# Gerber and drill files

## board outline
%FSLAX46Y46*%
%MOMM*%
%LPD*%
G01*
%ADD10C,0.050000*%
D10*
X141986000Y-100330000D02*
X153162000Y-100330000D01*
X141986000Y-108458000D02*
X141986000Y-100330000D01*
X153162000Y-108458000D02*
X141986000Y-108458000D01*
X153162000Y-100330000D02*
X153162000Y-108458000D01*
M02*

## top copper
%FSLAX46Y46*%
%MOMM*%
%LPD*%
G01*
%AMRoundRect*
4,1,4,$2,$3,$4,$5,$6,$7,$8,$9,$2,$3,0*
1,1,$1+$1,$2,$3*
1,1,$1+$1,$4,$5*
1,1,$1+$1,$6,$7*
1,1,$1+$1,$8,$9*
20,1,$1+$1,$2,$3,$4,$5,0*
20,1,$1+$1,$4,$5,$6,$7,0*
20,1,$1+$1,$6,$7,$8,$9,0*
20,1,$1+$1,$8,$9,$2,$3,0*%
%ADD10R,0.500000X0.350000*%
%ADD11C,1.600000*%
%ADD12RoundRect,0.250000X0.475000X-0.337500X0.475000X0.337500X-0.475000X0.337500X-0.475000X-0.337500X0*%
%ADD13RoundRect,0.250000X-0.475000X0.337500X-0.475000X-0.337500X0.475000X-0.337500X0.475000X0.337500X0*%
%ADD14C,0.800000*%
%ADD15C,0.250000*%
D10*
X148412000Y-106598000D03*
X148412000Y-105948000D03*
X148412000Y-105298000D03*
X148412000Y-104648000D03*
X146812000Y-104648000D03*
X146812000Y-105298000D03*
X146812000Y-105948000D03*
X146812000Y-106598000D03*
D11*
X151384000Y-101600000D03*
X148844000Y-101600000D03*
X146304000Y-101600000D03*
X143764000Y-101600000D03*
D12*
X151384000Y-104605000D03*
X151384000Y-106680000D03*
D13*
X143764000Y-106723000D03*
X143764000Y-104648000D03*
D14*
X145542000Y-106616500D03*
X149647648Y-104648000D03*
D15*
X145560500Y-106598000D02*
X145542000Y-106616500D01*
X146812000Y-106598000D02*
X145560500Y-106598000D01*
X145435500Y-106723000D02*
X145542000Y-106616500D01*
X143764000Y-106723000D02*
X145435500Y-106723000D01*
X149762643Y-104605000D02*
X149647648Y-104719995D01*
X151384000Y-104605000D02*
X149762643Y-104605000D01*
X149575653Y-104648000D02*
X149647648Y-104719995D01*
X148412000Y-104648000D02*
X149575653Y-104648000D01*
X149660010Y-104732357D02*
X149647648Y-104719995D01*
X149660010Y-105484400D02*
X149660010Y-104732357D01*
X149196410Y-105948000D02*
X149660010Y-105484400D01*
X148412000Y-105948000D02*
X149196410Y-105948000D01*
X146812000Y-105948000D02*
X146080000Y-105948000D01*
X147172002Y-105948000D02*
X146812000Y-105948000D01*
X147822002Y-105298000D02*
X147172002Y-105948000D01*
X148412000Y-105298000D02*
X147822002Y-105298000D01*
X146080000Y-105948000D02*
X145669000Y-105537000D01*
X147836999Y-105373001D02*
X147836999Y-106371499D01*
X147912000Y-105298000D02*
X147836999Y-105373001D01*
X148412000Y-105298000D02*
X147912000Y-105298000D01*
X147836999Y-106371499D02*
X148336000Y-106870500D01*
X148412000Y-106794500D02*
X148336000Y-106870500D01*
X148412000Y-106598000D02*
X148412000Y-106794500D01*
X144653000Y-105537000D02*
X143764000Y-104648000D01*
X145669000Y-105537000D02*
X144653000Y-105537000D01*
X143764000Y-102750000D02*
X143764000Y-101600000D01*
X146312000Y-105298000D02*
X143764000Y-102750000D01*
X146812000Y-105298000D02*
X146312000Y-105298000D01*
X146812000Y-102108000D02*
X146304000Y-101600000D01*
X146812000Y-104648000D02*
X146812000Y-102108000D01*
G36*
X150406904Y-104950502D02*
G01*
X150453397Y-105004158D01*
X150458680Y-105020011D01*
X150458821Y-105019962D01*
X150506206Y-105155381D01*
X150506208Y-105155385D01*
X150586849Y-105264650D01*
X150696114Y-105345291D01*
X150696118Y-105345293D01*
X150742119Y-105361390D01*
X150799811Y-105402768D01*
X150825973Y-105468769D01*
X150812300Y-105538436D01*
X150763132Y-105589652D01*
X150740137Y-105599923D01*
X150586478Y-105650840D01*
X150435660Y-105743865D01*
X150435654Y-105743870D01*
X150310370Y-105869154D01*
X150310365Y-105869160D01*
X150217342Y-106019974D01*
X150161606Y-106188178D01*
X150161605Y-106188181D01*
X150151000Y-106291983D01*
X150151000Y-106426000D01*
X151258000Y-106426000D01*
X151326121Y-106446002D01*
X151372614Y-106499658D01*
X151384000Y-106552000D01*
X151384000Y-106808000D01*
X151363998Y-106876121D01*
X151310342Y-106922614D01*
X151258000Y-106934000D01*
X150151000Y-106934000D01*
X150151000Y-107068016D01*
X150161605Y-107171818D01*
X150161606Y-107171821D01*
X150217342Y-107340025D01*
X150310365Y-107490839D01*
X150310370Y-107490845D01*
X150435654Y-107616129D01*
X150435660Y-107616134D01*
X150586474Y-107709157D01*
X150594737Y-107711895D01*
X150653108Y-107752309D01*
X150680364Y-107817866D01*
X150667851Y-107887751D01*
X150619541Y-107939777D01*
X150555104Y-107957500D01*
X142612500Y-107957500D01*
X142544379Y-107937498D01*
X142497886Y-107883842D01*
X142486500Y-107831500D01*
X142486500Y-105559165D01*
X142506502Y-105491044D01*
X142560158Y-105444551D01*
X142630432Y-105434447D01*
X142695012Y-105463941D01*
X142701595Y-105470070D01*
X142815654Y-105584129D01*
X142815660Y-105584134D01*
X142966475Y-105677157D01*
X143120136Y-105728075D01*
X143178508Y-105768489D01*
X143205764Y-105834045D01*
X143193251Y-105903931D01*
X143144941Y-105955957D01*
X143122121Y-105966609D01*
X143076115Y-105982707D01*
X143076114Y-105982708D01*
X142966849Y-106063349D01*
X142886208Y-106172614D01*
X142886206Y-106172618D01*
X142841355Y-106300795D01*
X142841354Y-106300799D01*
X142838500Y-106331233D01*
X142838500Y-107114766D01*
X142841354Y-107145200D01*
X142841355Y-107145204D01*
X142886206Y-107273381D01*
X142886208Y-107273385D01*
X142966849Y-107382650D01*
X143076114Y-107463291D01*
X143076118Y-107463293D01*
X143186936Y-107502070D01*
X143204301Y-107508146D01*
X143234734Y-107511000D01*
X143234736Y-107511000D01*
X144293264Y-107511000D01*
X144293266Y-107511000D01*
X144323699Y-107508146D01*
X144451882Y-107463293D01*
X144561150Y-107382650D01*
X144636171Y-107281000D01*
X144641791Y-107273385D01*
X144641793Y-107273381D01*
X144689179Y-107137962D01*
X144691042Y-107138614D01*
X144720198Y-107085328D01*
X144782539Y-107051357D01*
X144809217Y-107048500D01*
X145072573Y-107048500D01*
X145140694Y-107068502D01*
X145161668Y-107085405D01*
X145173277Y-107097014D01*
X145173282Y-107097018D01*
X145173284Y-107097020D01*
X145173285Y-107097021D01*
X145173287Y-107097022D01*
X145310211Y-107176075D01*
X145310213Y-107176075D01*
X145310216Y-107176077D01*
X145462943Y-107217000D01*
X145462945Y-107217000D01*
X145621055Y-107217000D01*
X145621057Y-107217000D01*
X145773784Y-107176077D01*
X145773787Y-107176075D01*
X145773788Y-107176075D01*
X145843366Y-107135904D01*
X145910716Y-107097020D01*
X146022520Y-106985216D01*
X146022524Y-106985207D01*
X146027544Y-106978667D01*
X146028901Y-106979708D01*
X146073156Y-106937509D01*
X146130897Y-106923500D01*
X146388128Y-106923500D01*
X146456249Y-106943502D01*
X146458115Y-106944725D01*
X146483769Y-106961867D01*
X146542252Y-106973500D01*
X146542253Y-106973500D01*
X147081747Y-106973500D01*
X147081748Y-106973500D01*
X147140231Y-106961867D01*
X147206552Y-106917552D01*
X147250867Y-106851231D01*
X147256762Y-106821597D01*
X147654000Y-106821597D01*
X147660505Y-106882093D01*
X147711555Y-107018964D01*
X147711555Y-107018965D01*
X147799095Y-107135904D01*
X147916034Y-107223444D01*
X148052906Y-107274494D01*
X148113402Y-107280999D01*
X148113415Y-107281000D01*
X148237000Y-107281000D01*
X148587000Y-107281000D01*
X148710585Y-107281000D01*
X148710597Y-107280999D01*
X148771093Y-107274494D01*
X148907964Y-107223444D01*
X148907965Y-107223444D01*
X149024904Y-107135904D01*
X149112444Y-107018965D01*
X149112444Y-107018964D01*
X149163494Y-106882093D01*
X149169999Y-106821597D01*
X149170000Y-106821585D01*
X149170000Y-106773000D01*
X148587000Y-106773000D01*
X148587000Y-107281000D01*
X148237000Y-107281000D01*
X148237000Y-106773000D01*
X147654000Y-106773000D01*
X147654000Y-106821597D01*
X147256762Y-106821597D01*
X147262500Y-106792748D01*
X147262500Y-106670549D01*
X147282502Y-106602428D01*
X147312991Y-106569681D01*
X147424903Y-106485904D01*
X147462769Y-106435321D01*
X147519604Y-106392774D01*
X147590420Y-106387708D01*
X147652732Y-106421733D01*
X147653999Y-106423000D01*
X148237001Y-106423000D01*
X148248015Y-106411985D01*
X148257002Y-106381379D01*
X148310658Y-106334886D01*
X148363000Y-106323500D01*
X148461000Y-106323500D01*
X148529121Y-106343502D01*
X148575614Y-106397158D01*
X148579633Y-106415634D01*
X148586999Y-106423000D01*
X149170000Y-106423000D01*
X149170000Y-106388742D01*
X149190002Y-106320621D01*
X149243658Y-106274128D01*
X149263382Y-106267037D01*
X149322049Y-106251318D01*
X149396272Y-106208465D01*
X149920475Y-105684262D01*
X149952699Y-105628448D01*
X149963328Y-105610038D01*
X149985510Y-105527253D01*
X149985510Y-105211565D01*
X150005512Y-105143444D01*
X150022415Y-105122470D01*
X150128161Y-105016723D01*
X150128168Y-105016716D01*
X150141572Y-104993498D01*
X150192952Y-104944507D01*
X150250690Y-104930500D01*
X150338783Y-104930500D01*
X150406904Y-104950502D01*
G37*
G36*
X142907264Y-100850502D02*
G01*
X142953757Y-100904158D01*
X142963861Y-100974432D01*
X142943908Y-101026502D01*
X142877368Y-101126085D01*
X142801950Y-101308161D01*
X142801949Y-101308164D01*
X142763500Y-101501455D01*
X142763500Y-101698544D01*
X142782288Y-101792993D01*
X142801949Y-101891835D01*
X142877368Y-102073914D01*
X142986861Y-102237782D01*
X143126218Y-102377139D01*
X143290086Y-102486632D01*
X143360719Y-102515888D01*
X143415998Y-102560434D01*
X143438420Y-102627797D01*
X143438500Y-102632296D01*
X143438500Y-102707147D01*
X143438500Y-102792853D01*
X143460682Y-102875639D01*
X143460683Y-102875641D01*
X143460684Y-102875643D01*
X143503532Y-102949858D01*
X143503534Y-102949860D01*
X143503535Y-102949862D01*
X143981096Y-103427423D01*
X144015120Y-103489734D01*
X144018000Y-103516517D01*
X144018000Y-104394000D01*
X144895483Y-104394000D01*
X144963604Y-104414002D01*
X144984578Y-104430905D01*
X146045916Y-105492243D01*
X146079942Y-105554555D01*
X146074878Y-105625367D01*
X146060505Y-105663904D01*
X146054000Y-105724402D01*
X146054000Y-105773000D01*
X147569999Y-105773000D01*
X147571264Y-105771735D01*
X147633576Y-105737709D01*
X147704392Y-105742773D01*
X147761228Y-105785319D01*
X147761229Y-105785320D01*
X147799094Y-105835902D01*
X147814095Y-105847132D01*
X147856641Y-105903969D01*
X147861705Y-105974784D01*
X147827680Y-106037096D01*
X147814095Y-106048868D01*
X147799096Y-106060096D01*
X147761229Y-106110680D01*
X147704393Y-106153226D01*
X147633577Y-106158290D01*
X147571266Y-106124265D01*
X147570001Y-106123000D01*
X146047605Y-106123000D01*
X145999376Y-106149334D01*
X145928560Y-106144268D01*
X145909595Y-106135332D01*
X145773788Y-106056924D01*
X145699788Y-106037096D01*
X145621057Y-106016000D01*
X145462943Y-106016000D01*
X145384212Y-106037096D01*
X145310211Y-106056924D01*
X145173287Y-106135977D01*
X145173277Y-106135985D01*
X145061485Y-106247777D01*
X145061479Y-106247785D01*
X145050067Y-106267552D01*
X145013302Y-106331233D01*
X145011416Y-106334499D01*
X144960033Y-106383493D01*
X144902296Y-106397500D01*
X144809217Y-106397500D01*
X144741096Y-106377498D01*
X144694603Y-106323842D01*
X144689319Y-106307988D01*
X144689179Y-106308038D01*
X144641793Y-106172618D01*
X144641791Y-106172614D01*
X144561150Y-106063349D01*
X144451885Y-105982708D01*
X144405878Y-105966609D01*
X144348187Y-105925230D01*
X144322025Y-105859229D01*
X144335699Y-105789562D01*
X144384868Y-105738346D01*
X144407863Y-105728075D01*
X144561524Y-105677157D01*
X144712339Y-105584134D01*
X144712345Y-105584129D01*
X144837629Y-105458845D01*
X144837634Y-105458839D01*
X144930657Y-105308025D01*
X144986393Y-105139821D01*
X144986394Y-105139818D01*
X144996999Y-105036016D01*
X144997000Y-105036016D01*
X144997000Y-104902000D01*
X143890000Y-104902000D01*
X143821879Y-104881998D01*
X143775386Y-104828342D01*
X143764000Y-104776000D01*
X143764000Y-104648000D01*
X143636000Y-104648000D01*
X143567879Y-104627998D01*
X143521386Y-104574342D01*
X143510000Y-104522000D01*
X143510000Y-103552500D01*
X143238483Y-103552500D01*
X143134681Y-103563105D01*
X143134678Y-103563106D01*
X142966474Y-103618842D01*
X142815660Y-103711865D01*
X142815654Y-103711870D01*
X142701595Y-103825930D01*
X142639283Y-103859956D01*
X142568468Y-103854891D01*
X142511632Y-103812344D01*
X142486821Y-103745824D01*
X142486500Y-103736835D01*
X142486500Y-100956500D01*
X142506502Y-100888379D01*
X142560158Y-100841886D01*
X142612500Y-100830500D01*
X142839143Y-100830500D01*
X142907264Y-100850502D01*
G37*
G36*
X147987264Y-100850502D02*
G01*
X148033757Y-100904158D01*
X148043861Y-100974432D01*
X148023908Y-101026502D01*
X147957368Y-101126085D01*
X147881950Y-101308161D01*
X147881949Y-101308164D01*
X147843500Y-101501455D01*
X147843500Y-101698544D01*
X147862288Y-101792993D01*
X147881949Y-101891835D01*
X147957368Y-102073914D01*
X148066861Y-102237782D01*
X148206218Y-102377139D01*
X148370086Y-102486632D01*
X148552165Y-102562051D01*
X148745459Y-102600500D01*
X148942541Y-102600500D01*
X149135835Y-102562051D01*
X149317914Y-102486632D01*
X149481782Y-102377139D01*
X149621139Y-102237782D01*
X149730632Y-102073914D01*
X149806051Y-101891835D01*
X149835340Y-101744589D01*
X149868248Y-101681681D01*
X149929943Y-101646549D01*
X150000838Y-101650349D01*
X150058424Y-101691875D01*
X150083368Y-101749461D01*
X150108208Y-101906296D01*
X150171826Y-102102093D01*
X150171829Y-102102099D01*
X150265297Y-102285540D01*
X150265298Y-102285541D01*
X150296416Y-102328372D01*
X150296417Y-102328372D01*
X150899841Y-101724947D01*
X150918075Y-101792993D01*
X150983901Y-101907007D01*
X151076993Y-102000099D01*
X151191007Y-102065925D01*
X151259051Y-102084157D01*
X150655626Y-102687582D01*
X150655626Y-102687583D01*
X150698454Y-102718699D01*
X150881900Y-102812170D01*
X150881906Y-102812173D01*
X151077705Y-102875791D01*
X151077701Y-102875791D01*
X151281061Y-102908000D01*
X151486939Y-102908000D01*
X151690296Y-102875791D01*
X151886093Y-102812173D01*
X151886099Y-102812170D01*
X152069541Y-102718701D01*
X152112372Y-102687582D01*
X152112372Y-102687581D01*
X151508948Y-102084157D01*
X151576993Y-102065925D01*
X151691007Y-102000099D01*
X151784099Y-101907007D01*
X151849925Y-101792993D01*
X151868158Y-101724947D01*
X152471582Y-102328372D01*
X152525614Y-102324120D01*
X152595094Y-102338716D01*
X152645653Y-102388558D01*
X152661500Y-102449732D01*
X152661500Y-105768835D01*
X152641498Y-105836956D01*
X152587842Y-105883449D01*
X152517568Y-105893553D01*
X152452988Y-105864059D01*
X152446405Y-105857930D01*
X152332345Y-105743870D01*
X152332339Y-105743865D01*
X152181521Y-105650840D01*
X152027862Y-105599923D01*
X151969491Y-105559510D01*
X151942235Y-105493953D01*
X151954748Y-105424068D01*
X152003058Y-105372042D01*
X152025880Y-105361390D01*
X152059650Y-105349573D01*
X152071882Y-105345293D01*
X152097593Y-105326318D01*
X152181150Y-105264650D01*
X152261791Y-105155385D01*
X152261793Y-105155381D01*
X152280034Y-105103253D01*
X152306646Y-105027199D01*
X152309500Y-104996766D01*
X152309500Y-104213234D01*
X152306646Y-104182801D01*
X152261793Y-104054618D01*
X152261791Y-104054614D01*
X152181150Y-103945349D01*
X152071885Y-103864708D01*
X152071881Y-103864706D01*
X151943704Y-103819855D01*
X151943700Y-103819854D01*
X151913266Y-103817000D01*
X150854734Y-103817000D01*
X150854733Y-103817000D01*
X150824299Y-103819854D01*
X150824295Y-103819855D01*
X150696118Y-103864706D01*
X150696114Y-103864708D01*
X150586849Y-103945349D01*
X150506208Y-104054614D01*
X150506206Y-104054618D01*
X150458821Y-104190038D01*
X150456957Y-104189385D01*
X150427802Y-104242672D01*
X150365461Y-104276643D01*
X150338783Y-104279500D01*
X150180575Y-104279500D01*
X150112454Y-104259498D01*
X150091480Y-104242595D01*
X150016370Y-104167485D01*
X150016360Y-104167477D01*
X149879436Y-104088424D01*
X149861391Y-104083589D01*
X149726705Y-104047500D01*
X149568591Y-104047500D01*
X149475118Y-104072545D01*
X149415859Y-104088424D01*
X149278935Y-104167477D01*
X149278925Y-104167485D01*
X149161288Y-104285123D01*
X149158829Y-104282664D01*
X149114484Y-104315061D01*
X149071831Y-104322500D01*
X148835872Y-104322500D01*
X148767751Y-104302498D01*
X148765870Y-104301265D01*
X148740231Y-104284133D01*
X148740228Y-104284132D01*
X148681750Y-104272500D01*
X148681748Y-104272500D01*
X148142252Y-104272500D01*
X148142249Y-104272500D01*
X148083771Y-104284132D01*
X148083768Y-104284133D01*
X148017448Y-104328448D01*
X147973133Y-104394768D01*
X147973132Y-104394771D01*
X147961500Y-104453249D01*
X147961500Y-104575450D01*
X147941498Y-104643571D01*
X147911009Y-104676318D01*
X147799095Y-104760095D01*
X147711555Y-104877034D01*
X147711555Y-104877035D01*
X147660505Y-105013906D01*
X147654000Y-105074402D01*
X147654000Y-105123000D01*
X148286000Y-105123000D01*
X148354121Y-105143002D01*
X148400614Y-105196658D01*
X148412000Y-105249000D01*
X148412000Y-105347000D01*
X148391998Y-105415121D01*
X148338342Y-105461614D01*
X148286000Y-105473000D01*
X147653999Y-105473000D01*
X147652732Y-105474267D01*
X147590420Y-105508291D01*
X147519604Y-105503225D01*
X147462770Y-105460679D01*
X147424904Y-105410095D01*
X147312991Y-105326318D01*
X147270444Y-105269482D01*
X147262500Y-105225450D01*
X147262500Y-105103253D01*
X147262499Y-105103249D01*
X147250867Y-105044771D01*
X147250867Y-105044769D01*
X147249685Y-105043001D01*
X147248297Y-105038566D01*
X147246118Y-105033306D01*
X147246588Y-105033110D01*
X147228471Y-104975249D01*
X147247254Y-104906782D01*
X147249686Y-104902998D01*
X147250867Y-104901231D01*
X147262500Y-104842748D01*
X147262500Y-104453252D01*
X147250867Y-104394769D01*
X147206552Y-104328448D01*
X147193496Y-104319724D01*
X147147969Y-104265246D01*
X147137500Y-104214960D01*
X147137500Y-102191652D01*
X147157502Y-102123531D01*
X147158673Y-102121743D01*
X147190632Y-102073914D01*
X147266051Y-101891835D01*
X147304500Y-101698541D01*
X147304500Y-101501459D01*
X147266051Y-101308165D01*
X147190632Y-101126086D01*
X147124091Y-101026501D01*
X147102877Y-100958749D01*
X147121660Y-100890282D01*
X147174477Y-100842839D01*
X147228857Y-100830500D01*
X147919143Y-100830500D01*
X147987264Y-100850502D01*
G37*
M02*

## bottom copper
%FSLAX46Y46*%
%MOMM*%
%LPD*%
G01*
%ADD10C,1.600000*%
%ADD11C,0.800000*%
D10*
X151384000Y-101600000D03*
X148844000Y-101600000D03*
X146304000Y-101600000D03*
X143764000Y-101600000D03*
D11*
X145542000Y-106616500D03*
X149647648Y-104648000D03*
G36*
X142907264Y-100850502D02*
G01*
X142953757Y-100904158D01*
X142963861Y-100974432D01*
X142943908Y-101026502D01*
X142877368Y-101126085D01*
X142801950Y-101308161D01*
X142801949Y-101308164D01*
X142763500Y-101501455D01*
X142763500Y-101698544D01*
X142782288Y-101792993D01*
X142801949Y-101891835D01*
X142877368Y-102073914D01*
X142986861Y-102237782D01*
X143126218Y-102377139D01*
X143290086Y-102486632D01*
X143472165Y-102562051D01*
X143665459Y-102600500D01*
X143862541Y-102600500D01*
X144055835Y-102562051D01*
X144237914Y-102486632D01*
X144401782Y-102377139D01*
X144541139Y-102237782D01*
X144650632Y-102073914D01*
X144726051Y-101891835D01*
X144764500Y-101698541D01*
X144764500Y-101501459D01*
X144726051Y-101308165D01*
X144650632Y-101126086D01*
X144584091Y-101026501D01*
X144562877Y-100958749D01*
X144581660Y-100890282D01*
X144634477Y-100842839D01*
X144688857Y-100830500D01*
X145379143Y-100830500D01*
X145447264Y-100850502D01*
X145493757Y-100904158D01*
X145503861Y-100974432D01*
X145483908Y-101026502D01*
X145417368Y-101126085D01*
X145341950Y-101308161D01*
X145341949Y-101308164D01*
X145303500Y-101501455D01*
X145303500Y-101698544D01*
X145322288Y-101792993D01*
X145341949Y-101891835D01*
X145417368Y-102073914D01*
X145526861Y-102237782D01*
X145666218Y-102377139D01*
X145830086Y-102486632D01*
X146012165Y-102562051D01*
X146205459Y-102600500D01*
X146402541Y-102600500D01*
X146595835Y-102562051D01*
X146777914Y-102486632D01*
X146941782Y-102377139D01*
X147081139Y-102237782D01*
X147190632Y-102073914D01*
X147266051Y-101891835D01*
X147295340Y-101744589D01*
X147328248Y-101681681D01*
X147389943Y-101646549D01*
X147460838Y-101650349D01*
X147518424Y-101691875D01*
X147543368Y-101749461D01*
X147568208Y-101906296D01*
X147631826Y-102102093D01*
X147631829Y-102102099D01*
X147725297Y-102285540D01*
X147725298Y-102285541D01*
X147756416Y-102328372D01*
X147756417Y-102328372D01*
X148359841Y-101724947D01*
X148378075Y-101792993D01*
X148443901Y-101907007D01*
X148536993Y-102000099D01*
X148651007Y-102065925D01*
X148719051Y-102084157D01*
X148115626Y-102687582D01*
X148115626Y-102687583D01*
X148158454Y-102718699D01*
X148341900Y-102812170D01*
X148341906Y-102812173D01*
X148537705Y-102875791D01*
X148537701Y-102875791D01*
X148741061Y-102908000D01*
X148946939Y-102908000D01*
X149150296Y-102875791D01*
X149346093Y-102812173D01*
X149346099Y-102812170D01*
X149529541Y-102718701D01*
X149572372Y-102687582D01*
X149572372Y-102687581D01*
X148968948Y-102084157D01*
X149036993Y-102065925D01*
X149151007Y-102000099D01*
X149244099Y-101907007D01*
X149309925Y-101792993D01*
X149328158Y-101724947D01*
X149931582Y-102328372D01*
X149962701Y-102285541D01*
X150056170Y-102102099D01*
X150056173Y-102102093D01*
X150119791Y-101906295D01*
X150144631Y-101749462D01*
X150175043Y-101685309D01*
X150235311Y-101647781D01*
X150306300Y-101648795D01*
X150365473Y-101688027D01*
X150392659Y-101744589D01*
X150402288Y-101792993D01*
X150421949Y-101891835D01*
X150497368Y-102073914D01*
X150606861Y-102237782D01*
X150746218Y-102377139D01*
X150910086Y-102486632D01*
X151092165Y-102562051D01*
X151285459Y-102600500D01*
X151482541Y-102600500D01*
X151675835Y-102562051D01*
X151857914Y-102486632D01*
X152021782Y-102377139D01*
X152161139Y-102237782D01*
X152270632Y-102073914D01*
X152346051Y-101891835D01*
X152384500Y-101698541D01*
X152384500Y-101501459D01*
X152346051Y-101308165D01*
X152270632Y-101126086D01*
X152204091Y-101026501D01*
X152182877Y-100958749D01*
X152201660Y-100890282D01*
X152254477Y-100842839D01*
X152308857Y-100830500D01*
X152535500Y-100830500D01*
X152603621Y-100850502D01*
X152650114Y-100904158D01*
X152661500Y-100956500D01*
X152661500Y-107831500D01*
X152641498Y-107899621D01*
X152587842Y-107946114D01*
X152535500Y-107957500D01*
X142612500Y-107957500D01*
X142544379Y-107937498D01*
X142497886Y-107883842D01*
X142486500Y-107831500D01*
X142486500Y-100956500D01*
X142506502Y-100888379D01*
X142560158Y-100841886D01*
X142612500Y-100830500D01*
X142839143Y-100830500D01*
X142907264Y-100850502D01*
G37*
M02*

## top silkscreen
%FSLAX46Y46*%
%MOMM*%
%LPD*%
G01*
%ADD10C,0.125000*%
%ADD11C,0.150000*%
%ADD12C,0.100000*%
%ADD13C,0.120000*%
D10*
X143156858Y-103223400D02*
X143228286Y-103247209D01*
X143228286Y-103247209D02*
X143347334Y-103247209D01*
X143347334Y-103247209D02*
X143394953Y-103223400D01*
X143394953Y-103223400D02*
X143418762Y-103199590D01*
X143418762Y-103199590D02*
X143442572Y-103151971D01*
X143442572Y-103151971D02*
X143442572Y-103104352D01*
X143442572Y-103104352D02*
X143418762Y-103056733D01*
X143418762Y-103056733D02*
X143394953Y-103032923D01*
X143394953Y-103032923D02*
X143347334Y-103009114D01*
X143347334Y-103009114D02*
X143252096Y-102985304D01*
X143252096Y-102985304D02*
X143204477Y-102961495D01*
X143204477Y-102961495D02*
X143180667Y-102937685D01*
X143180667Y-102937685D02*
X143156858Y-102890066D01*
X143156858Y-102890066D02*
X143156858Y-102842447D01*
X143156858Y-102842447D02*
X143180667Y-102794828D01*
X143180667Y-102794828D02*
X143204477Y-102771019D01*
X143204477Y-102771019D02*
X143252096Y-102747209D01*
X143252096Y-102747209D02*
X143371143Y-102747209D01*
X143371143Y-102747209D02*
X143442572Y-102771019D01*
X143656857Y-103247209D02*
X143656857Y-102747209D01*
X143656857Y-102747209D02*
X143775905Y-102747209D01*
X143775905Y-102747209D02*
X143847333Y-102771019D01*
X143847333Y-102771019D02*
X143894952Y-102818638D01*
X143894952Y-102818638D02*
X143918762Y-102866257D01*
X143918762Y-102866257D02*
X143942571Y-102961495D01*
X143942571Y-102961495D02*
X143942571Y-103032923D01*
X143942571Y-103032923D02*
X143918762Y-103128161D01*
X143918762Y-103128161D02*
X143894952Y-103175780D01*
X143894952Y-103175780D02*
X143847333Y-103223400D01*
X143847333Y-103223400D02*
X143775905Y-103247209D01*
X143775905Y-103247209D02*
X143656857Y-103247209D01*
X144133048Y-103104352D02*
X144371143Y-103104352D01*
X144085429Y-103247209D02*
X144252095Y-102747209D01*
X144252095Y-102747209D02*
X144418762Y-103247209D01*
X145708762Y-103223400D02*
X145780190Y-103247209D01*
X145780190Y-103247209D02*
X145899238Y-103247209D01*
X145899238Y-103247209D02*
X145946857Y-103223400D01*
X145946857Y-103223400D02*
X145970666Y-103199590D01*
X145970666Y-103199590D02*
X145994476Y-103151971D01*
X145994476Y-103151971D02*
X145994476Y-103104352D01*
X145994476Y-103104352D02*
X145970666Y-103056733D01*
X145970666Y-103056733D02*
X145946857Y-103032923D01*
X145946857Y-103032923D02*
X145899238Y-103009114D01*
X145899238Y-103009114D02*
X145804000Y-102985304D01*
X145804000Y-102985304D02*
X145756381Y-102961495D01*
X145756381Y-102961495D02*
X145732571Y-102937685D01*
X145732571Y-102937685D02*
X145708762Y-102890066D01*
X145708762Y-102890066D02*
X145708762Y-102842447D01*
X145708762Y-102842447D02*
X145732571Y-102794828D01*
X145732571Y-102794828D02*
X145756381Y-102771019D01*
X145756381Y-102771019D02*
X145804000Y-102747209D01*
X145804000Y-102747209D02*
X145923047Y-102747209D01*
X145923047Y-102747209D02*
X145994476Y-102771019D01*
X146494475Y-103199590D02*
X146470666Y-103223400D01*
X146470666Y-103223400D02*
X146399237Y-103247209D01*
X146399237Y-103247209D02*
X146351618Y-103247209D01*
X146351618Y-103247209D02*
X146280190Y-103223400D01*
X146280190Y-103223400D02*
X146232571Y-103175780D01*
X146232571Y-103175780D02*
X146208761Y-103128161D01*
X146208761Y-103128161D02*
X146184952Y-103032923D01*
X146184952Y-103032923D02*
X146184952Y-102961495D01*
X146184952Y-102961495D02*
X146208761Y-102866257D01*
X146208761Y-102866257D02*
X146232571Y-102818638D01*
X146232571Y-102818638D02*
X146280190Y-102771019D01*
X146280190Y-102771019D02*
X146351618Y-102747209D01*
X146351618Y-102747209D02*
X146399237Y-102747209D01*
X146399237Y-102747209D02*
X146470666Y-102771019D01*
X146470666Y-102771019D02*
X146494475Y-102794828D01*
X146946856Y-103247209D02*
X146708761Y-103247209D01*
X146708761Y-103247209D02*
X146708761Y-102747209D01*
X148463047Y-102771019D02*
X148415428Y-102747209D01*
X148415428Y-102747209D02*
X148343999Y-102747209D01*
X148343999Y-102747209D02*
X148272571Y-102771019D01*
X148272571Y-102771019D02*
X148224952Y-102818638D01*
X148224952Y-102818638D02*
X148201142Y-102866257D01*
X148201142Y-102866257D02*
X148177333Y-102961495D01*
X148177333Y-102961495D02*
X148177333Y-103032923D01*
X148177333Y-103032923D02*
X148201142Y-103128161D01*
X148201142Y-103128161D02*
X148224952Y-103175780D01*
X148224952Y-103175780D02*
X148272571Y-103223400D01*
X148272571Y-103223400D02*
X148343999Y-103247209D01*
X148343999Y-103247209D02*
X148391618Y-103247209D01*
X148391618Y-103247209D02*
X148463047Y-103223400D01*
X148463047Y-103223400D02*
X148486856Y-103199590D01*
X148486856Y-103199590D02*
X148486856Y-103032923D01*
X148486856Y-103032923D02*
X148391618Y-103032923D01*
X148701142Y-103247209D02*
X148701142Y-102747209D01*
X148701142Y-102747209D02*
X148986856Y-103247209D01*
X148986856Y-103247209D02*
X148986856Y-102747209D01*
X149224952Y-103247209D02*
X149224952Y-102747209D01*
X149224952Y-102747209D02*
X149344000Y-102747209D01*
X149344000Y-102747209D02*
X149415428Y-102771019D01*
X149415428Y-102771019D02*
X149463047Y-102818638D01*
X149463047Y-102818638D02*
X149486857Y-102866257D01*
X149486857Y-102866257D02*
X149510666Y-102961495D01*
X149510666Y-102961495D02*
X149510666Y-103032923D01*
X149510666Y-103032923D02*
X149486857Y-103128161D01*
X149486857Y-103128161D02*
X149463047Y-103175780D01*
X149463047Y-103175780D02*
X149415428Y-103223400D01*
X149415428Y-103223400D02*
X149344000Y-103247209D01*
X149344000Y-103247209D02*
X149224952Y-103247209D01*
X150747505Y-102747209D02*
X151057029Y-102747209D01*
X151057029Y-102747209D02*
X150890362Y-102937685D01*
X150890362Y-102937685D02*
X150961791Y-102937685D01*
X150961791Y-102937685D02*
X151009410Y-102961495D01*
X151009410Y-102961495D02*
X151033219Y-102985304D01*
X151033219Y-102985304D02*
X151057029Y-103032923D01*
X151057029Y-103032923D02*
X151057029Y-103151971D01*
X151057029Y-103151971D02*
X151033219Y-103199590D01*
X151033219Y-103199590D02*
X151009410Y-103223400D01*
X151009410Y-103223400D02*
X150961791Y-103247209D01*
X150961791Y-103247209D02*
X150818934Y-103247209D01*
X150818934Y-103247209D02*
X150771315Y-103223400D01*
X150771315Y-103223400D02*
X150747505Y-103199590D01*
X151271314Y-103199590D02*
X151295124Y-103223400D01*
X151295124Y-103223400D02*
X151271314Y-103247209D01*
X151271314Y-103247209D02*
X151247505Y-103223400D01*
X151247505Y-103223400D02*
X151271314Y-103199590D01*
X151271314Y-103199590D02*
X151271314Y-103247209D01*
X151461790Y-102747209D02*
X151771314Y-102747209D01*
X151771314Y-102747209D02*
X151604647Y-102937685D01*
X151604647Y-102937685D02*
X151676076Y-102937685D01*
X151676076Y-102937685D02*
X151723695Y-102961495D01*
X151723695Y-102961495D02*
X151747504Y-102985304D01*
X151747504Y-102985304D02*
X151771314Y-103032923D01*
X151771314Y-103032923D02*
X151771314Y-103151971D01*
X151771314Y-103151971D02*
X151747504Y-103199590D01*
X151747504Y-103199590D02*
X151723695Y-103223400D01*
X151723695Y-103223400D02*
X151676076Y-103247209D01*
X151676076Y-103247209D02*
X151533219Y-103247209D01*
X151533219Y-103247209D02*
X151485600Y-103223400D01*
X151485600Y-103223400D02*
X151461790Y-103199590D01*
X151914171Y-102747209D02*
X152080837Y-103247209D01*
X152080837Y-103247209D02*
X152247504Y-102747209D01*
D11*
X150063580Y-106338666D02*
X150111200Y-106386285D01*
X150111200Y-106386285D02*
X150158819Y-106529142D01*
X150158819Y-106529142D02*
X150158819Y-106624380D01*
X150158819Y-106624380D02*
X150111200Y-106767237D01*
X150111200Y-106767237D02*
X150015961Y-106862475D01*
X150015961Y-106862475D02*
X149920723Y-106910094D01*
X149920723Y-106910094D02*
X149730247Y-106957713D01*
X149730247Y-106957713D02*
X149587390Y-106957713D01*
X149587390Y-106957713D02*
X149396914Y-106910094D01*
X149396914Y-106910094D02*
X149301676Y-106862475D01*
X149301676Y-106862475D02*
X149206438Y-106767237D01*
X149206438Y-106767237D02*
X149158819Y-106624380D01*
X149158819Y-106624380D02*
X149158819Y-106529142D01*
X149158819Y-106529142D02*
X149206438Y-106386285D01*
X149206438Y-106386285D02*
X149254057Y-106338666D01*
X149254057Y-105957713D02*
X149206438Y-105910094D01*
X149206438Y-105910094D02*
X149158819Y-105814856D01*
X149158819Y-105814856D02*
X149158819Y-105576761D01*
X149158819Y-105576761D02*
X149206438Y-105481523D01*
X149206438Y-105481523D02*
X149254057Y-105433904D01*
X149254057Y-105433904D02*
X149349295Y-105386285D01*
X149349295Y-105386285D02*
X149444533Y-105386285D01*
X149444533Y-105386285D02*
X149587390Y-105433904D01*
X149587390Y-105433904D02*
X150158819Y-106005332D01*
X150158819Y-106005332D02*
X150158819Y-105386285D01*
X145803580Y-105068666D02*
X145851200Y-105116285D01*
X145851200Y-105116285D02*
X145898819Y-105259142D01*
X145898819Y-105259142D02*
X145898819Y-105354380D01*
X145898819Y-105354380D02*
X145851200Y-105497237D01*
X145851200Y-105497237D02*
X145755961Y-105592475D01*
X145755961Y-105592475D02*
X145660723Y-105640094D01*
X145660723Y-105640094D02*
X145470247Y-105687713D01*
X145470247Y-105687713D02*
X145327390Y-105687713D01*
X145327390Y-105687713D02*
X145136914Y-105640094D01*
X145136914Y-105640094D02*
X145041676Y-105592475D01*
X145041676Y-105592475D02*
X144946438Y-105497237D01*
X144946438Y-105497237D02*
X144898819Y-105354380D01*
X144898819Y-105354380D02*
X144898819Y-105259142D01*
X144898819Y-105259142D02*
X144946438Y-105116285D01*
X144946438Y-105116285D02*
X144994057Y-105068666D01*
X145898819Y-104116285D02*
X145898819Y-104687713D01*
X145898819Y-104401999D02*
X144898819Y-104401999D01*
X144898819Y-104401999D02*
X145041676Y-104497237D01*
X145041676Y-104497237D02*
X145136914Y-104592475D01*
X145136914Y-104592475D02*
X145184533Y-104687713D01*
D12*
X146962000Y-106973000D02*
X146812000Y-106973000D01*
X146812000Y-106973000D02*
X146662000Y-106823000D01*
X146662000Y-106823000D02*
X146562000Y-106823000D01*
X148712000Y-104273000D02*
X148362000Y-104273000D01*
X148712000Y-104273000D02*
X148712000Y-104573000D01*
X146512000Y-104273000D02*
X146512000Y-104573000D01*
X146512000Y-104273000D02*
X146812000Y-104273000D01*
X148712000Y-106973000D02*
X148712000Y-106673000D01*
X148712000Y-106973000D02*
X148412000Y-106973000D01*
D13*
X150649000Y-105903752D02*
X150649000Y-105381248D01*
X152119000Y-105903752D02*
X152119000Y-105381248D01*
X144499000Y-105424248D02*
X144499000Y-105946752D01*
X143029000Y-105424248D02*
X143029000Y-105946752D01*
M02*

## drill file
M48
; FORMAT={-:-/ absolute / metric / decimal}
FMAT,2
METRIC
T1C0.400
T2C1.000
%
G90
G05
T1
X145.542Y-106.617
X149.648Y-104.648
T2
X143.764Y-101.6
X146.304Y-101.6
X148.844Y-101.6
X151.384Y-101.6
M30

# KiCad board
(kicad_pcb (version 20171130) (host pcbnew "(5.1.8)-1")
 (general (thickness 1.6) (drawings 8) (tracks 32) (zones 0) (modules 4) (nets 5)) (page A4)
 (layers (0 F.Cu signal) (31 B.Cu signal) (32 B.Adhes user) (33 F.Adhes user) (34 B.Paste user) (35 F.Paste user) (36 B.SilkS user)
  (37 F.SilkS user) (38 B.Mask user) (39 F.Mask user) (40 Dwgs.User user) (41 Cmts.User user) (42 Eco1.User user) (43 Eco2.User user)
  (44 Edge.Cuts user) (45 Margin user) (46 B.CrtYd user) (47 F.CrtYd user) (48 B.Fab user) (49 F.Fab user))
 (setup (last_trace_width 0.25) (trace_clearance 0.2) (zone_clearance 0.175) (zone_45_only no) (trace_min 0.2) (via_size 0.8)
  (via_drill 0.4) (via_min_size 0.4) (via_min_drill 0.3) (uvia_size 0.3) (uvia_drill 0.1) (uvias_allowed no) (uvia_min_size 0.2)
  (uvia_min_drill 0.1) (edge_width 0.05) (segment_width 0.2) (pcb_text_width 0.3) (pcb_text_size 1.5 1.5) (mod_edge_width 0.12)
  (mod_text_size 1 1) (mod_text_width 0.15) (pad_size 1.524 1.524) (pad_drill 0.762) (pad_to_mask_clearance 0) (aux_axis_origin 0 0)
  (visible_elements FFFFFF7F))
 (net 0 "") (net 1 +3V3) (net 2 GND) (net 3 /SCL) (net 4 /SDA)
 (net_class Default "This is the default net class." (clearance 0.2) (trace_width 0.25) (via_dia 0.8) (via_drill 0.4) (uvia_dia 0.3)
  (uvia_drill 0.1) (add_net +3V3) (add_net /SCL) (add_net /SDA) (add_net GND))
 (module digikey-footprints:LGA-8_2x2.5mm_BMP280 (layer F.Cu) (at 147.612 105.623 180)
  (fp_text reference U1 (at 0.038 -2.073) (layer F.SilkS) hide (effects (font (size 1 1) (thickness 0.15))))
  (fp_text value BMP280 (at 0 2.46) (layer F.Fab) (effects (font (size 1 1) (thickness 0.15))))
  (fp_line (start 0.65 -1.35) (end 0.8 -1.35) (layer F.SilkS) (width 0.1))
  (fp_line (start 0.8 -1.35) (end 0.95 -1.2) (layer F.SilkS) (width 0.1))
  (fp_line (start 0.95 -1.2) (end 1.05 -1.2) (layer F.SilkS) (width 0.1))
  (fp_line (start -1.1 1.35) (end -0.75 1.35) (layer F.SilkS) (width 0.1))
  (fp_line (start -1.1 1.35) (end -1.1 1.05) (layer F.SilkS) (width 0.1))
  (fp_line (start 1.1 1.35) (end 1.1 1.05) (layer F.SilkS) (width 0.1))
  (fp_line (start 1.1 1.35) (end 0.8 1.35) (layer F.SilkS) (width 0.1))
  (fp_line (start -1.1 -1.35) (end -1.1 -1.05) (layer F.SilkS) (width 0.1))
  (fp_line (start -1.1 -1.35) (end -0.8 -1.35) (layer F.SilkS) (width 0.1))
  (pad 8 smd rect (at -0.8 -0.975 180) (size 0.5 0.35) (layers F.Cu F.Paste F.Mask) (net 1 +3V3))
  (pad 7 smd rect (at -0.8 -0.325 180) (size 0.5 0.35) (layers F.Cu F.Paste F.Mask) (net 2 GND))
  (pad 6 smd rect (at -0.8 0.325 180) (size 0.5 0.35) (layers F.Cu F.Paste F.Mask) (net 1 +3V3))
  (pad 5 smd rect (at -0.8 0.975 180) (size 0.5 0.35) (layers F.Cu F.Paste F.Mask) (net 2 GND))
  (pad 4 smd rect (at 0.8 0.975 180) (size 0.5 0.35) (layers F.Cu F.Paste F.Mask) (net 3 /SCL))
  (pad 3 smd rect (at 0.8 0.325 180) (size 0.5 0.35) (layers F.Cu F.Paste F.Mask) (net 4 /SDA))
  (pad 2 smd rect (at 0.8 -0.325 180) (size 0.5 0.35) (layers F.Cu F.Paste F.Mask) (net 1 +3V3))
  (pad 1 smd rect (at 0.8 -0.975 180) (size 0.5 0.35) (layers F.Cu F.Paste F.Mask) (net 2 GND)))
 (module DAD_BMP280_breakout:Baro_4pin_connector (layer F.Cu) (at 151.384 101.6 180)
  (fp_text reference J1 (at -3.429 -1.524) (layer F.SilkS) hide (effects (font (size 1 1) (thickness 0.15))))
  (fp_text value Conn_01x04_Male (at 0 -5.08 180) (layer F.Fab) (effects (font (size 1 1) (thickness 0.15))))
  (pad 1 thru_hole circle (at 0 0 180) (size 1.6 1.6) (drill 1) (layers *.Cu *.Mask) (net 1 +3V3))
  (pad 2 thru_hole circle (at 2.54 0 180) (size 1.6 1.6) (drill 1) (layers *.Cu *.Mask) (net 2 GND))
  (pad 3 thru_hole circle (at 5.08 0 180) (size 1.6 1.6) (drill 1) (layers *.Cu *.Mask) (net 3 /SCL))
  (pad 4 thru_hole circle (at 7.62 0 180) (size 1.6 1.6) (drill 1) (layers *.Cu *.Mask) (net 4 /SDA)))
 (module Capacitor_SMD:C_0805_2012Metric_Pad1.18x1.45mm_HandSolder (layer F.Cu) (at 151.384 105.6425 90)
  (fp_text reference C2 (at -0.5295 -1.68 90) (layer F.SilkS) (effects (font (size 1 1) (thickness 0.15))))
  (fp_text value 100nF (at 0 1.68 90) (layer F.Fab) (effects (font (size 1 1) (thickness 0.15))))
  (fp_line (start -0.261252 -0.735) (end 0.261252 -0.735) (layer F.SilkS) (width 0.12))
  (fp_line (start -0.261252 0.735) (end 0.261252 0.735) (layer F.SilkS) (width 0.12))
  (pad 2 smd roundrect (at 1.0375 0 90) (size 1.175 1.45) (layers F.Cu F.Paste F.Mask) (roundrect_rratio 0.2127659574468085) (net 2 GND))
  (pad 1 smd roundrect (at -1.0375 0 90) (size 1.175 1.45) (layers F.Cu F.Paste F.Mask) (roundrect_rratio 0.2127659574468085) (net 1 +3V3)))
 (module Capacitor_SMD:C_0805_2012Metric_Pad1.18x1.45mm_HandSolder (layer F.Cu) (at 143.764 105.6855 270)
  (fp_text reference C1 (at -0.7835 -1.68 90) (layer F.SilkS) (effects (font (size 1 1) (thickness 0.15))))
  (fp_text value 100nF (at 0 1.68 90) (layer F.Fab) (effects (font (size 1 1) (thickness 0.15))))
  (fp_line (start -0.261252 -0.735) (end 0.261252 -0.735) (layer F.SilkS) (width 0.12))
  (fp_line (start -0.261252 0.735) (end 0.261252 0.735) (layer F.SilkS) (width 0.12))
  (pad 2 smd roundrect (at 1.0375 0 270) (size 1.175 1.45) (layers F.Cu F.Paste F.Mask) (roundrect_rratio 0.2127659574468085) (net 2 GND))
  (pad 1 smd roundrect (at -1.0375 0 270) (size 1.175 1.45) (layers F.Cu F.Paste F.Mask) (roundrect_rratio 0.2127659574468085) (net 1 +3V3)))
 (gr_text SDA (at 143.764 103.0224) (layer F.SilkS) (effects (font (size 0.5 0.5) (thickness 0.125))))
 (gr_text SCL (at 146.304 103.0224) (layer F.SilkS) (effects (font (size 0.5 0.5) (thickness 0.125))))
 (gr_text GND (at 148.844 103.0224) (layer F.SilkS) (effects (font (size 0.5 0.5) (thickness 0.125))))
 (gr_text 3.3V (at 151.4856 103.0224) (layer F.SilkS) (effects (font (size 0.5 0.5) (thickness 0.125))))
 (gr_line (start 141.986 100.33) (end 153.162 100.33) (layer Edge.Cuts) (width 0.05))
 (gr_line (start 141.986 108.458) (end 141.986 100.33) (layer Edge.Cuts) (width 0.05))
 (gr_line (start 153.162 108.458) (end 141.986 108.458) (layer Edge.Cuts) (width 0.05))
 (gr_line (start 153.162 100.33) (end 153.162 108.458) (layer Edge.Cuts) (width 0.05))
 (via (at 145.542 106.6165) (size 0.8) (drill 0.4) (layers F.Cu B.Cu) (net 2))
 (segment (start 145.5605 106.598) (end 145.542 106.6165) (width 0.25) (layer F.Cu) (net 2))
 (segment (start 146.812 106.598) (end 145.5605 106.598) (width 0.25) (layer F.Cu) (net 2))
 (segment (start 145.4355 106.723) (end 145.542 106.6165) (width 0.25) (layer F.Cu) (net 2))
 (segment (start 143.764 106.723) (end 145.4355 106.723) (width 0.25) (layer F.Cu) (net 2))
 (via (at 149.647648 104.648) (size 0.8) (drill 0.4) (layers F.Cu B.Cu) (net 2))
 (segment (start 149.762643 104.605) (end 149.647648 104.719995) (width 0.25) (layer F.Cu) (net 2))
 (segment (start 151.384 104.605) (end 149.762643 104.605) (width 0.25) (layer F.Cu) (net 2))
 (segment (start 149.575653 104.648) (end 149.647648 104.719995) (width 0.25) (layer F.Cu) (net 2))
 (segment (start 148.412 104.648) (end 149.575653 104.648) (width 0.25) (layer F.Cu) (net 2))
 (segment (start 149.66001 104.732357) (end 149.647648 104.719995) (width 0.25) (layer F.Cu) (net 2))
 (segment (start 149.66001 105.4844) (end 149.66001 104.732357) (width 0.25) (layer F.Cu) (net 2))
 (segment (start 149.19641 105.948) (end 149.66001 105.4844) (width 0.25) (layer F.Cu) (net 2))
 (segment (start 148.412 105.948) (end 149.19641 105.948) (width 0.25) (layer F.Cu) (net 2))
 (segment (start 146.812 105.948) (end 146.08 105.948) (width 0.25) (layer F.Cu) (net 1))
 (segment (start 147.172002 105.948) (end 146.812 105.948) (width 0.25) (layer F.Cu) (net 1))
 (segment (start 147.822002 105.298) (end 147.172002 105.948) (width 0.25) (layer F.Cu) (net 1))
 (segment (start 148.412 105.298) (end 147.822002 105.298) (width 0.25) (layer F.Cu) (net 1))
 (segment (start 146.08 105.948) (end 145.669 105.537) (width 0.25) (layer F.Cu) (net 1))
 (segment (start 147.836999 105.373001) (end 147.836999 106.371499) (width 0.25) (layer F.Cu) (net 1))
 (segment (start 147.912 105.298) (end 147.836999 105.373001) (width 0.25) (layer F.Cu) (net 1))
 (segment (start 148.412 105.298) (end 147.912 105.298) (width 0.25) (layer F.Cu) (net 1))
 (segment (start 147.836999 106.371499) (end 148.336 106.8705) (width 0.25) (layer F.Cu) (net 1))
 (segment (start 148.412 106.7945) (end 148.336 106.8705) (width 0.25) (layer F.Cu) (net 1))
 (segment (start 148.412 106.598) (end 148.412 106.7945) (width 0.25) (layer F.Cu) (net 1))
 (segment (start 144.653 105.537) (end 143.764 104.648) (width 0.25) (layer F.Cu) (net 1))
 (segment (start 145.669 105.537) (end 144.653 105.537) (width 0.25) (layer F.Cu) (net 1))
 (segment (start 143.764 102.75) (end 143.764 101.6) (width 0.25) (layer F.Cu) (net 4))
 (segment (start 146.312 105.298) (end 143.764 102.75) (width 0.25) (layer F.Cu) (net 4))
 (segment (start 146.812 105.298) (end 146.312 105.298) (width 0.25) (layer F.Cu) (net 4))
 (segment (start 146.812 102.108) (end 146.304 101.6) (width 0.25) (layer F.Cu) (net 3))
 (segment (start 146.812 104.648) (end 146.812 102.108) (width 0.25) (layer F.Cu) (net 3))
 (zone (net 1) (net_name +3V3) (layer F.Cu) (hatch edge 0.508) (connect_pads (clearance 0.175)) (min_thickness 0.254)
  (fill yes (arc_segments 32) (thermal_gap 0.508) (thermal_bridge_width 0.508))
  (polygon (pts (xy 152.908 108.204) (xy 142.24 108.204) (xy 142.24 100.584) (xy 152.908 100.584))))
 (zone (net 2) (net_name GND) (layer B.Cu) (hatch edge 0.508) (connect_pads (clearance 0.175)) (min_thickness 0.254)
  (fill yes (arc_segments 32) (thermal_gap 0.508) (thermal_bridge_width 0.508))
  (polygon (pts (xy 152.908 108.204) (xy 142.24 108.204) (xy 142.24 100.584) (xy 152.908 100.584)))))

